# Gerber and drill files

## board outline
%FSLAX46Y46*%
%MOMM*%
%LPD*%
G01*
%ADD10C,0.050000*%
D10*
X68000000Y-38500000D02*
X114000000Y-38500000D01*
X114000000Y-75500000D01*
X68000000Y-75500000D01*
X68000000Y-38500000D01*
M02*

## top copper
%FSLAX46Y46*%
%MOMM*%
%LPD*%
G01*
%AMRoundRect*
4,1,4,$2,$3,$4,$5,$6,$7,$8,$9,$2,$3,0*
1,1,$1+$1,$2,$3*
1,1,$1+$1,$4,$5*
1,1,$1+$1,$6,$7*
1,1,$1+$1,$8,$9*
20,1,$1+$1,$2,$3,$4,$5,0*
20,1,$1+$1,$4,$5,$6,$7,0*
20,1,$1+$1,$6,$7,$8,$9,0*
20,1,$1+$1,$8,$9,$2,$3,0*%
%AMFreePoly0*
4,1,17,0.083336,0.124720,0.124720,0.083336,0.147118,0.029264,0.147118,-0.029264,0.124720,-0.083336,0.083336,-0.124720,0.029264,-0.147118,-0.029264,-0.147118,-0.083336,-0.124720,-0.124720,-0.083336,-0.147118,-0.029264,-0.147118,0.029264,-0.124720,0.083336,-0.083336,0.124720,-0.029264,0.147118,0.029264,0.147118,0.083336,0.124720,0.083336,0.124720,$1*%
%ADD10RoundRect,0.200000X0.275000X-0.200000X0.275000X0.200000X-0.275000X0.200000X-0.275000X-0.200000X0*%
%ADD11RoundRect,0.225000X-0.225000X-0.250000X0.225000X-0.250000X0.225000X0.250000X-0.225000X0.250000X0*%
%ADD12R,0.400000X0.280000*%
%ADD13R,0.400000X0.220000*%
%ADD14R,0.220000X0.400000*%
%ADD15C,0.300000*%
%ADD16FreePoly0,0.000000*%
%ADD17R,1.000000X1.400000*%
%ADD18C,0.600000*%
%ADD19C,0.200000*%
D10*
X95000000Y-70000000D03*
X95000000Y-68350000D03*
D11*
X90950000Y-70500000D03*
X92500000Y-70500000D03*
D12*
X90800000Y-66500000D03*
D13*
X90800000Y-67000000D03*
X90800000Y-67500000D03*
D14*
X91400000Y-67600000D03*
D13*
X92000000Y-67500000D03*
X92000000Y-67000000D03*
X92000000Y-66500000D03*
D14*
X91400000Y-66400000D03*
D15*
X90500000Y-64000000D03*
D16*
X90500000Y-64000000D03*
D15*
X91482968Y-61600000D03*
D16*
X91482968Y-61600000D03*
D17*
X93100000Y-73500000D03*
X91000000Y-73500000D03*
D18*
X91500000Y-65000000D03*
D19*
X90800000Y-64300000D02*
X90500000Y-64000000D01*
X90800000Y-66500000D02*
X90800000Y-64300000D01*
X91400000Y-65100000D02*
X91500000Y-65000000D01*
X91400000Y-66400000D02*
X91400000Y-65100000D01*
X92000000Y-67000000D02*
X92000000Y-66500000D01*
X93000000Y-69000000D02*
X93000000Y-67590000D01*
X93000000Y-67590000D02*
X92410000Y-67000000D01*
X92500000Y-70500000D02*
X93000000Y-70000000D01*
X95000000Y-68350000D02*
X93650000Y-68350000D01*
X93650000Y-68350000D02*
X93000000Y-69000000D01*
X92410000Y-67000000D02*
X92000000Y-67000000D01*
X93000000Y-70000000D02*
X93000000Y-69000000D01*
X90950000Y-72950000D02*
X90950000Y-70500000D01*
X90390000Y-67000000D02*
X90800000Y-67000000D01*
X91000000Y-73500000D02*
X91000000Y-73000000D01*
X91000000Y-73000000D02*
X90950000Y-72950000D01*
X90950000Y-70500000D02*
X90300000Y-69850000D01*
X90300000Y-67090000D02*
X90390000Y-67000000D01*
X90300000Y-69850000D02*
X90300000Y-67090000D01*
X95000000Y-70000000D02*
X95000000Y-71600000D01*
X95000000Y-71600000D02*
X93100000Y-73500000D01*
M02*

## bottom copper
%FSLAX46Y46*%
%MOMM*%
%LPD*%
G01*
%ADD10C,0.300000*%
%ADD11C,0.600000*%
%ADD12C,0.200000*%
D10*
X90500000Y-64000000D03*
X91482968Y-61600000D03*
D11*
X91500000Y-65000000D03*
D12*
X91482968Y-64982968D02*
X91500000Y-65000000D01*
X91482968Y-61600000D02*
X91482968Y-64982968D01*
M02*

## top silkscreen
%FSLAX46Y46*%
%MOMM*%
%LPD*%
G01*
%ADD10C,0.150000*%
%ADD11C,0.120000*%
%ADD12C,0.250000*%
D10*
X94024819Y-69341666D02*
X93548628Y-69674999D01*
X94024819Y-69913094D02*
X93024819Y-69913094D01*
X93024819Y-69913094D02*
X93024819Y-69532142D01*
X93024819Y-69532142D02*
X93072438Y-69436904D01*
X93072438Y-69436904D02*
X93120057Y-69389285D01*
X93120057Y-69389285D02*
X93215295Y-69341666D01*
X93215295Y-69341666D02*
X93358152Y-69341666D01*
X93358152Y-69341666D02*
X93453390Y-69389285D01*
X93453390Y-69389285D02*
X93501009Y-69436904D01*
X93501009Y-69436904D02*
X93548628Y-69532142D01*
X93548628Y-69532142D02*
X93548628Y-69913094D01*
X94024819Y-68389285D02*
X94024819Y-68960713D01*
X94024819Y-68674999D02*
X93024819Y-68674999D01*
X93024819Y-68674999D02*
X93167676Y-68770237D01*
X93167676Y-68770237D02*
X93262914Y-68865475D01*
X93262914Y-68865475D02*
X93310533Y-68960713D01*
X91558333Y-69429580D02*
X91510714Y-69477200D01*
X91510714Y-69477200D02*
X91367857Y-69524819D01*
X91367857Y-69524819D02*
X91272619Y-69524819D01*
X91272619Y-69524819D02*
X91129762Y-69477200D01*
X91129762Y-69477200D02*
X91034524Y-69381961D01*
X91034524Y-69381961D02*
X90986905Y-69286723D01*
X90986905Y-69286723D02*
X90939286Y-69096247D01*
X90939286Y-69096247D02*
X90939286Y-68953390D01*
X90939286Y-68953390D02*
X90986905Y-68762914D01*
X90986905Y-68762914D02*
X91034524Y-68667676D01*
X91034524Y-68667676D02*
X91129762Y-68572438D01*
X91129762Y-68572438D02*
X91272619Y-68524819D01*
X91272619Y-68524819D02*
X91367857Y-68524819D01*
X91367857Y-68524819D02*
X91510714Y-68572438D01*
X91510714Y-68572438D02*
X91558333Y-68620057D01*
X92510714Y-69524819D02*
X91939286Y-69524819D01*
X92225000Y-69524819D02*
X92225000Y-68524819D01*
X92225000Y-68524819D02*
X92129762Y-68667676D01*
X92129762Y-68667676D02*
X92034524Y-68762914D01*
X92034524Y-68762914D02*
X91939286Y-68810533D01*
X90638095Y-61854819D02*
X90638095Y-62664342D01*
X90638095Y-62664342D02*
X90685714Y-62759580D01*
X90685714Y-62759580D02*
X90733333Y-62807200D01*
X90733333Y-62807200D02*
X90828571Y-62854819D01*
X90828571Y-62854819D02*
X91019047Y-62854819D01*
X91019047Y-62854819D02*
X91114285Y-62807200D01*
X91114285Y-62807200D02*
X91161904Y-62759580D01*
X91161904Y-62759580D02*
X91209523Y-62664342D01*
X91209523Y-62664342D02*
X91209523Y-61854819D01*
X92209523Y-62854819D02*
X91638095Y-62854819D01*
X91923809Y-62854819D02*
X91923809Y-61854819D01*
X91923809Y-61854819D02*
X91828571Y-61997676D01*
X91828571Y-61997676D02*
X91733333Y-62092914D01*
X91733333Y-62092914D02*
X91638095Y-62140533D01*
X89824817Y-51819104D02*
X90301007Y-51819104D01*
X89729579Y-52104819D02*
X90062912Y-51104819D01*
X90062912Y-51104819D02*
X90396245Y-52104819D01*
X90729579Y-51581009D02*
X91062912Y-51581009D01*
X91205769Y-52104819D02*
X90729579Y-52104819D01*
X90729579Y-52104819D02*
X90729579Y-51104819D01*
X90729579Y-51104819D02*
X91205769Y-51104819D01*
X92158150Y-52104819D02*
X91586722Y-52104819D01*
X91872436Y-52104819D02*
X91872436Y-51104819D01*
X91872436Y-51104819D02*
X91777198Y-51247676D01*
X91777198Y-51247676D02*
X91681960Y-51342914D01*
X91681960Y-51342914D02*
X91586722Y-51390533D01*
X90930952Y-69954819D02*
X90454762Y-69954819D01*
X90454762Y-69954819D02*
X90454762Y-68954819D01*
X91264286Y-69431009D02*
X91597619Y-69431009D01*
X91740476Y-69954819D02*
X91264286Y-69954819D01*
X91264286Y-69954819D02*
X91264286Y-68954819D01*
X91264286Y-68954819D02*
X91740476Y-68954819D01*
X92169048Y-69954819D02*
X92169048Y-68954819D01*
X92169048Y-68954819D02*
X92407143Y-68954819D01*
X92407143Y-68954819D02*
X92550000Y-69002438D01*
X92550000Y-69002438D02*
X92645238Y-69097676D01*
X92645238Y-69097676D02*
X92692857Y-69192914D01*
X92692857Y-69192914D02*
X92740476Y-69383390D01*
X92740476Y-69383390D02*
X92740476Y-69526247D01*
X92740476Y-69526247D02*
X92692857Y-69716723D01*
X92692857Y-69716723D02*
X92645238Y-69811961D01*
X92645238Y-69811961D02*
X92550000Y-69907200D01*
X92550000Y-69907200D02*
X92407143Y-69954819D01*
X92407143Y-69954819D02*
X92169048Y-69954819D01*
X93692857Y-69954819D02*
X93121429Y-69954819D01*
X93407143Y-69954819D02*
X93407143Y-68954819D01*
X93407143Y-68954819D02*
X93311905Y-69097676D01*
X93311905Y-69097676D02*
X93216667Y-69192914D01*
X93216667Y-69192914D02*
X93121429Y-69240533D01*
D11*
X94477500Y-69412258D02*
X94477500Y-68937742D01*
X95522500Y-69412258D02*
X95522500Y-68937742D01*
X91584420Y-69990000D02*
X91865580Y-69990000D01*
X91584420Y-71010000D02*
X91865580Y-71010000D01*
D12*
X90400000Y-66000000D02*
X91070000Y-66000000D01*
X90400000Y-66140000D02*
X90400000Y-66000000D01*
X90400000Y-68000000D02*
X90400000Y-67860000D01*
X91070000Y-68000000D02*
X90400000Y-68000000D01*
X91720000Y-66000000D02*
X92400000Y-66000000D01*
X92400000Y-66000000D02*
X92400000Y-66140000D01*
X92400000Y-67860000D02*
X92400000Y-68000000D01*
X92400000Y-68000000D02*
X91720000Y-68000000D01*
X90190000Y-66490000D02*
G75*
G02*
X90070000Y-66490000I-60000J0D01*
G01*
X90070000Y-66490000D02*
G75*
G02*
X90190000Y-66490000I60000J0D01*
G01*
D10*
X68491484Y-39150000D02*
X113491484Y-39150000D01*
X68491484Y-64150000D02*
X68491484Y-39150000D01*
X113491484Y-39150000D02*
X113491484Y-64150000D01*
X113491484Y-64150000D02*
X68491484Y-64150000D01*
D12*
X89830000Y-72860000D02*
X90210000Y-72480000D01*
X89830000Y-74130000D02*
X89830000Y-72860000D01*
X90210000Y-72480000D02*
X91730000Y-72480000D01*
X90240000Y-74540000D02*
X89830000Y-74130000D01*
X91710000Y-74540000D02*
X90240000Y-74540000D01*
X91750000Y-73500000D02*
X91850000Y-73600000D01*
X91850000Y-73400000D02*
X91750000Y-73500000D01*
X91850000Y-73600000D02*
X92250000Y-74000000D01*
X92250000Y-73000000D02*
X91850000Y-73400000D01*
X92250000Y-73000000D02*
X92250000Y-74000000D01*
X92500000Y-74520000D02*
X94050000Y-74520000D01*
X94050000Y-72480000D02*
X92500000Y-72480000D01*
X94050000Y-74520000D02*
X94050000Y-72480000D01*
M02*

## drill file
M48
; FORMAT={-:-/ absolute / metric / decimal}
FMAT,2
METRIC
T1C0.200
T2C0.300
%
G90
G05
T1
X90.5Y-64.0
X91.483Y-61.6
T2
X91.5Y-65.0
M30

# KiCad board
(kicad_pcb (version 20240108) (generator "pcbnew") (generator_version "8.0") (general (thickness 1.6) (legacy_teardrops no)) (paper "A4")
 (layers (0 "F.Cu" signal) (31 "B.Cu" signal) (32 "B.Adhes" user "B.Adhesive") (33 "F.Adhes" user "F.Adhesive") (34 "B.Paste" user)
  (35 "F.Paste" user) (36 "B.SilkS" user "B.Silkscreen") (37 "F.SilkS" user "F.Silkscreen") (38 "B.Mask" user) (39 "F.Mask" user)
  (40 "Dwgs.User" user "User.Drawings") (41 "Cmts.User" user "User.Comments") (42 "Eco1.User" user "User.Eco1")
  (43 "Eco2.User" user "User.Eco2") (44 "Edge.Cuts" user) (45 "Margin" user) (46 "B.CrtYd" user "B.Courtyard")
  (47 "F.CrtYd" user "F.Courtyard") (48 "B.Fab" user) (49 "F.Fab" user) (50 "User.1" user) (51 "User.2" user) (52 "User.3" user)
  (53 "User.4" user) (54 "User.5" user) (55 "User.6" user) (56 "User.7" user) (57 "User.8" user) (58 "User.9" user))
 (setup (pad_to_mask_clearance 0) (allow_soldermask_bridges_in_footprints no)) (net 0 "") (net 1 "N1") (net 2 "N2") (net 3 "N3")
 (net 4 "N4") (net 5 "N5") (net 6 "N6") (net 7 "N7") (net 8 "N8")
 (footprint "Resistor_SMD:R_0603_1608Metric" (layer "F.Cu") (at 95 69.175 90)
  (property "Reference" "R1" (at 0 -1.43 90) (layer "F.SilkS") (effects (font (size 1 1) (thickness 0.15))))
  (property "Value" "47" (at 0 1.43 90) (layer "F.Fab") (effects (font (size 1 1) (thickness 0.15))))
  (fp_line (start -0.237258 -0.5225) (end 0.237258 -0.5225) (stroke (width 0.12) (type solid)) (layer "F.SilkS"))
  (fp_line (start -0.237258 0.5225) (end 0.237258 0.5225) (stroke (width 0.12) (type solid)) (layer "F.SilkS"))
  (pad "1" smd roundrect (at -0.825 0 90) (size 0.8 0.95) (layers "F.Cu" "F.Paste" "F.Mask") (roundrect_rratio 0.25) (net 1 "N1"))
  (pad "2" smd roundrect (at 0.825 0 90) (size 0.8 0.95) (layers "F.Cu" "F.Paste" "F.Mask") (roundrect_rratio 0.25) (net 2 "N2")))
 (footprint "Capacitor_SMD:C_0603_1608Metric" (layer "F.Cu") (at 91.725 70.5)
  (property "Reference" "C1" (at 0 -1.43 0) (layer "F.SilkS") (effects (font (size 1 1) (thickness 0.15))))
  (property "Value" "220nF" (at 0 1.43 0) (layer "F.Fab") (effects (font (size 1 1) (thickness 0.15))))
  (fp_line (start -0.14058 -0.51) (end 0.14058 -0.51) (stroke (width 0.12) (type solid)) (layer "F.SilkS"))
  (fp_line (start -0.14058 0.51) (end 0.14058 0.51) (stroke (width 0.12) (type solid)) (layer "F.SilkS"))
  (pad "1" smd roundrect (at -0.775 0) (size 0.9 0.95) (layers "F.Cu" "F.Paste" "F.Mask") (roundrect_rratio 0.25) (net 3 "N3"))
  (pad "2" smd roundrect (at 0.775 0) (size 0.9 0.95) (layers "F.Cu" "F.Paste" "F.Mask") (roundrect_rratio 0.25) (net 2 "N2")))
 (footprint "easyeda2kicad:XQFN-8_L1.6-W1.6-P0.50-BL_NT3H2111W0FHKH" (layer "F.Cu") (at 91.4 67)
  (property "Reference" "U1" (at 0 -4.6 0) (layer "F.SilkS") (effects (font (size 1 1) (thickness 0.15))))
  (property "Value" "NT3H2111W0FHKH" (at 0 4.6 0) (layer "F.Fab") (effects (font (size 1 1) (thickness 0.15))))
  (fp_line (start -1 -1) (end -0.33 -1) (stroke (width 0.25) (type solid)) (layer "F.SilkS"))
  (fp_line (start -1 -0.86) (end -1 -1) (stroke (width 0.25) (type solid)) (layer "F.SilkS"))
  (fp_line (start -1 1) (end -1 0.86) (stroke (width 0.25) (type solid)) (layer "F.SilkS"))
  (fp_line (start -0.33 1) (end -1 1) (stroke (width 0.25) (type solid)) (layer "F.SilkS"))
  (fp_line (start 0.32 -1) (end 1 -1) (stroke (width 0.25) (type solid)) (layer "F.SilkS"))
  (fp_line (start 1 -1) (end 1 -0.86) (stroke (width 0.25) (type solid)) (layer "F.SilkS"))
  (fp_line (start 1 0.86) (end 1 1) (stroke (width 0.25) (type solid)) (layer "F.SilkS"))
  (fp_line (start 1 1) (end 0.32 1) (stroke (width 0.25) (type solid)) (layer "F.SilkS"))
  (fp_circle (center -1.27 -0.51) (end -1.21 -0.51) (stroke (width 0.25) (type solid)) (fill none) (layer "F.SilkS"))
  (pad "1" smd rect (at -0.6 -0.5) (size 0.4 0.28) (layers "F.Cu" "F.Paste" "F.Mask") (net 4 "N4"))
  (pad "2" smd rect (at -0.6 0) (size 0.4 0.22) (layers "F.Cu" "F.Paste" "F.Mask") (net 3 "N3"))
  (pad "3" smd rect (at -0.6 0.5) (size 0.4 0.22) (layers "F.Cu" "F.Paste" "F.Mask") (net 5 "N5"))
  (pad "4" smd rect (at 0 0.6 90) (size 0.4 0.22) (layers "F.Cu" "F.Paste" "F.Mask") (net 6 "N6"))
  (pad "5" smd rect (at 0.6 0.5) (size 0.4 0.22) (layers "F.Cu" "F.Paste" "F.Mask") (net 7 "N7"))
  (pad "6" smd rect (at 0.6 0) (size 0.4 0.22) (layers "F.Cu" "F.Paste" "F.Mask") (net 2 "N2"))
  (pad "7" smd rect (at 0.6 -0.5) (size 0.4 0.22) (layers "F.Cu" "F.Paste" "F.Mask") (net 2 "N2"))
  (pad "8" smd rect (at 0 -0.6 90) (size 0.4 0.22) (layers "F.Cu" "F.Paste" "F.Mask") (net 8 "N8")))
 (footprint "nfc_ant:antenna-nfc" (layer "F.Cu") (at 68.491484 39.15)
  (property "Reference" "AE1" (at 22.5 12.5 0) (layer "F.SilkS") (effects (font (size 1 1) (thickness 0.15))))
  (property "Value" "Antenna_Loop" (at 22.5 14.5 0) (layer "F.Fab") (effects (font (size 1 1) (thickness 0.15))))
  (fp_line (start 0 0) (end 45 0) (stroke (width 0.15) (type solid)) (layer "F.SilkS"))
  (fp_line (start 0 25) (end 0 0) (stroke (width 0.15) (type solid)) (layer "F.SilkS"))
  (fp_line (start 45 0) (end 45 25) (stroke (width 0.15) (type solid)) (layer "F.SilkS"))
  (fp_line (start 45 25) (end 0 25) (stroke (width 0.15) (type solid)) (layer "F.SilkS"))
  (pad "1" thru_hole circle (at 22.008516 24.85) (size 0.3 0.3) (drill 0.2) (layers "*.Cu" "*.Mask") (remove_unused_layers no) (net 4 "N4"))
  (pad "1" smd custom (at 22.008516 24.85) (size 0.3 0.3) (layers "F.Cu") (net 4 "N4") (zone_connect 0) (thermal_bridge_angle 90)
   (options (clearance outline) (anchor circle)) (primitives))
  (pad "2" thru_hole circle (at 22.991484 22.45) (size 0.3 0.3) (drill 0.2) (layers "*.Cu" "*.Mask") (remove_unused_layers no) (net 8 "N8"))
  (pad "2" smd custom (at 22.991484 22.45) (size 0.3 0.3) (layers "F.Cu") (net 8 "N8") (zone_connect 0) (thermal_bridge_angle 90)
   (options (clearance outline) (anchor circle)) (primitives)))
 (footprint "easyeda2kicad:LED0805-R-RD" (layer "F.Cu") (at 92.05 73.5)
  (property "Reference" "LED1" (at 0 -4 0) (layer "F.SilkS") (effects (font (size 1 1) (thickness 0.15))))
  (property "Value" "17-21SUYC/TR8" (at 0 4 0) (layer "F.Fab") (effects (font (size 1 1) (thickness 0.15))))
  (fp_line (start -2.22 -0.64) (end -1.84 -1.02) (stroke (width 0.25) (type solid)) (layer "F.SilkS"))
  (fp_line (start -2.22 0.63) (end -2.22 -0.64) (stroke (width 0.25) (type solid)) (layer "F.SilkS"))
  (fp_line (start -1.84 -1.02) (end -0.32 -1.02) (stroke (width 0.25) (type solid)) (layer "F.SilkS"))
  (fp_line (start -1.81 1.04) (end -2.22 0.63) (stroke (width 0.25) (type solid)) (layer "F.SilkS"))
  (fp_line (start -0.34 1.04) (end -1.81 1.04) (stroke (width 0.25) (type solid)) (layer "F.SilkS"))
  (fp_line (start -0.3 0) (end -0.2 0.1) (stroke (width 0.25) (type solid)) (layer "F.SilkS"))
  (fp_line (start -0.2 -0.1) (end -0.3 0) (stroke (width 0.25) (type solid)) (layer "F.SilkS"))
  (fp_line (start -0.2 0.1) (end 0.2 0.5) (stroke (width 0.25) (type solid)) (layer "F.SilkS"))
  (fp_line (start 0.2 -0.5) (end -0.2 -0.1) (stroke (width 0.25) (type solid)) (layer "F.SilkS"))
  (fp_line (start 0.2 -0.5) (end 0.2 0.5) (stroke (width 0.25) (type solid)) (layer "F.SilkS"))
  (fp_line (start 0.45 1.02) (end 2 1.02) (stroke (width 0.25) (type solid)) (layer "F.SilkS"))
  (fp_line (start 2 -1.02) (end 0.45 -1.02) (stroke (width 0.25) (type solid)) (layer "F.SilkS"))
  (fp_line (start 2 1.02) (end 2 -1.02) (stroke (width 0.25) (type solid)) (layer "F.SilkS"))
  (pad "1" smd rect (at 1.05 0 180) (size 1 1.4) (layers "F.Cu" "F.Paste" "F.Mask") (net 1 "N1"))
  (pad "2" smd rect (at -1.05 0 180) (size 1 1.4) (layers "F.Cu" "F.Paste" "F.Mask") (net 3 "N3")))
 (gr_rect (start 68 38.5) (end 114 75.5) (stroke (width 0.05) (type default)) (fill none) (layer "Edge.Cuts"))
 (segment (start 90.8 64.3) (end 90.5 64) (width 0.2) (layer "F.Cu") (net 4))
 (segment (start 90.8 66.5) (end 90.8 64.3) (width 0.2) (layer "F.Cu") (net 4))
 (segment (start 91.4 65.1) (end 91.5 65) (width 0.2) (layer "F.Cu") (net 8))
 (segment (start 91.4 66.4) (end 91.4 65.1) (width 0.2) (layer "F.Cu") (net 8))
 (via (at 91.5 65) (size 0.6) (drill 0.3) (layers "F.Cu" "B.Cu") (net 8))
 (segment (start 91.482968 64.982968) (end 91.5 65) (width 0.2) (layer "B.Cu") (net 8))
 (segment (start 91.482968 61.6) (end 91.482968 64.982968) (width 0.2) (layer "B.Cu") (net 8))
 (segment (start 92 67) (end 92 66.5) (width 0.2) (layer "F.Cu") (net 2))
 (segment (start 93 69) (end 93 67.59) (width 0.2) (layer "F.Cu") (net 2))
 (segment (start 93 67.59) (end 92.41 67) (width 0.2) (layer "F.Cu") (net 2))
 (segment (start 92.5 70.5) (end 93 70) (width 0.2) (layer "F.Cu") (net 2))
 (segment (start 95 68.35) (end 93.65 68.35) (width 0.2) (layer "F.Cu") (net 2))
 (segment (start 93.65 68.35) (end 93 69) (width 0.2) (layer "F.Cu") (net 2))
 (segment (start 92.41 67) (end 92 67) (width 0.2) (layer "F.Cu") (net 2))
 (segment (start 93 70) (end 93 69) (width 0.2) (layer "F.Cu") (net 2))
 (segment (start 90.95 72.95) (end 90.95 70.5) (width 0.2) (layer "F.Cu") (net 3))
 (segment (start 90.39 67) (end 90.8 67) (width 0.2) (layer "F.Cu") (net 3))
 (segment (start 91 73.5) (end 91 73) (width 0.2) (layer "F.Cu") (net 3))
 (segment (start 91 73) (end 90.95 72.95) (width 0.2) (layer "F.Cu") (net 3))
 (segment (start 90.95 70.5) (end 90.3 69.85) (width 0.2) (layer "F.Cu") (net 3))
 (segment (start 90.3 67.09) (end 90.39 67) (width 0.2) (layer "F.Cu") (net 3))
 (segment (start 90.3 69.85) (end 90.3 67.09) (width 0.2) (layer "F.Cu") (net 3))
 (segment (start 95 70) (end 95 71.6) (width 0.2) (layer "F.Cu") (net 1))
 (segment (start 95 71.6) (end 93.1 73.5) (width 0.2) (layer "F.Cu") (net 1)))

